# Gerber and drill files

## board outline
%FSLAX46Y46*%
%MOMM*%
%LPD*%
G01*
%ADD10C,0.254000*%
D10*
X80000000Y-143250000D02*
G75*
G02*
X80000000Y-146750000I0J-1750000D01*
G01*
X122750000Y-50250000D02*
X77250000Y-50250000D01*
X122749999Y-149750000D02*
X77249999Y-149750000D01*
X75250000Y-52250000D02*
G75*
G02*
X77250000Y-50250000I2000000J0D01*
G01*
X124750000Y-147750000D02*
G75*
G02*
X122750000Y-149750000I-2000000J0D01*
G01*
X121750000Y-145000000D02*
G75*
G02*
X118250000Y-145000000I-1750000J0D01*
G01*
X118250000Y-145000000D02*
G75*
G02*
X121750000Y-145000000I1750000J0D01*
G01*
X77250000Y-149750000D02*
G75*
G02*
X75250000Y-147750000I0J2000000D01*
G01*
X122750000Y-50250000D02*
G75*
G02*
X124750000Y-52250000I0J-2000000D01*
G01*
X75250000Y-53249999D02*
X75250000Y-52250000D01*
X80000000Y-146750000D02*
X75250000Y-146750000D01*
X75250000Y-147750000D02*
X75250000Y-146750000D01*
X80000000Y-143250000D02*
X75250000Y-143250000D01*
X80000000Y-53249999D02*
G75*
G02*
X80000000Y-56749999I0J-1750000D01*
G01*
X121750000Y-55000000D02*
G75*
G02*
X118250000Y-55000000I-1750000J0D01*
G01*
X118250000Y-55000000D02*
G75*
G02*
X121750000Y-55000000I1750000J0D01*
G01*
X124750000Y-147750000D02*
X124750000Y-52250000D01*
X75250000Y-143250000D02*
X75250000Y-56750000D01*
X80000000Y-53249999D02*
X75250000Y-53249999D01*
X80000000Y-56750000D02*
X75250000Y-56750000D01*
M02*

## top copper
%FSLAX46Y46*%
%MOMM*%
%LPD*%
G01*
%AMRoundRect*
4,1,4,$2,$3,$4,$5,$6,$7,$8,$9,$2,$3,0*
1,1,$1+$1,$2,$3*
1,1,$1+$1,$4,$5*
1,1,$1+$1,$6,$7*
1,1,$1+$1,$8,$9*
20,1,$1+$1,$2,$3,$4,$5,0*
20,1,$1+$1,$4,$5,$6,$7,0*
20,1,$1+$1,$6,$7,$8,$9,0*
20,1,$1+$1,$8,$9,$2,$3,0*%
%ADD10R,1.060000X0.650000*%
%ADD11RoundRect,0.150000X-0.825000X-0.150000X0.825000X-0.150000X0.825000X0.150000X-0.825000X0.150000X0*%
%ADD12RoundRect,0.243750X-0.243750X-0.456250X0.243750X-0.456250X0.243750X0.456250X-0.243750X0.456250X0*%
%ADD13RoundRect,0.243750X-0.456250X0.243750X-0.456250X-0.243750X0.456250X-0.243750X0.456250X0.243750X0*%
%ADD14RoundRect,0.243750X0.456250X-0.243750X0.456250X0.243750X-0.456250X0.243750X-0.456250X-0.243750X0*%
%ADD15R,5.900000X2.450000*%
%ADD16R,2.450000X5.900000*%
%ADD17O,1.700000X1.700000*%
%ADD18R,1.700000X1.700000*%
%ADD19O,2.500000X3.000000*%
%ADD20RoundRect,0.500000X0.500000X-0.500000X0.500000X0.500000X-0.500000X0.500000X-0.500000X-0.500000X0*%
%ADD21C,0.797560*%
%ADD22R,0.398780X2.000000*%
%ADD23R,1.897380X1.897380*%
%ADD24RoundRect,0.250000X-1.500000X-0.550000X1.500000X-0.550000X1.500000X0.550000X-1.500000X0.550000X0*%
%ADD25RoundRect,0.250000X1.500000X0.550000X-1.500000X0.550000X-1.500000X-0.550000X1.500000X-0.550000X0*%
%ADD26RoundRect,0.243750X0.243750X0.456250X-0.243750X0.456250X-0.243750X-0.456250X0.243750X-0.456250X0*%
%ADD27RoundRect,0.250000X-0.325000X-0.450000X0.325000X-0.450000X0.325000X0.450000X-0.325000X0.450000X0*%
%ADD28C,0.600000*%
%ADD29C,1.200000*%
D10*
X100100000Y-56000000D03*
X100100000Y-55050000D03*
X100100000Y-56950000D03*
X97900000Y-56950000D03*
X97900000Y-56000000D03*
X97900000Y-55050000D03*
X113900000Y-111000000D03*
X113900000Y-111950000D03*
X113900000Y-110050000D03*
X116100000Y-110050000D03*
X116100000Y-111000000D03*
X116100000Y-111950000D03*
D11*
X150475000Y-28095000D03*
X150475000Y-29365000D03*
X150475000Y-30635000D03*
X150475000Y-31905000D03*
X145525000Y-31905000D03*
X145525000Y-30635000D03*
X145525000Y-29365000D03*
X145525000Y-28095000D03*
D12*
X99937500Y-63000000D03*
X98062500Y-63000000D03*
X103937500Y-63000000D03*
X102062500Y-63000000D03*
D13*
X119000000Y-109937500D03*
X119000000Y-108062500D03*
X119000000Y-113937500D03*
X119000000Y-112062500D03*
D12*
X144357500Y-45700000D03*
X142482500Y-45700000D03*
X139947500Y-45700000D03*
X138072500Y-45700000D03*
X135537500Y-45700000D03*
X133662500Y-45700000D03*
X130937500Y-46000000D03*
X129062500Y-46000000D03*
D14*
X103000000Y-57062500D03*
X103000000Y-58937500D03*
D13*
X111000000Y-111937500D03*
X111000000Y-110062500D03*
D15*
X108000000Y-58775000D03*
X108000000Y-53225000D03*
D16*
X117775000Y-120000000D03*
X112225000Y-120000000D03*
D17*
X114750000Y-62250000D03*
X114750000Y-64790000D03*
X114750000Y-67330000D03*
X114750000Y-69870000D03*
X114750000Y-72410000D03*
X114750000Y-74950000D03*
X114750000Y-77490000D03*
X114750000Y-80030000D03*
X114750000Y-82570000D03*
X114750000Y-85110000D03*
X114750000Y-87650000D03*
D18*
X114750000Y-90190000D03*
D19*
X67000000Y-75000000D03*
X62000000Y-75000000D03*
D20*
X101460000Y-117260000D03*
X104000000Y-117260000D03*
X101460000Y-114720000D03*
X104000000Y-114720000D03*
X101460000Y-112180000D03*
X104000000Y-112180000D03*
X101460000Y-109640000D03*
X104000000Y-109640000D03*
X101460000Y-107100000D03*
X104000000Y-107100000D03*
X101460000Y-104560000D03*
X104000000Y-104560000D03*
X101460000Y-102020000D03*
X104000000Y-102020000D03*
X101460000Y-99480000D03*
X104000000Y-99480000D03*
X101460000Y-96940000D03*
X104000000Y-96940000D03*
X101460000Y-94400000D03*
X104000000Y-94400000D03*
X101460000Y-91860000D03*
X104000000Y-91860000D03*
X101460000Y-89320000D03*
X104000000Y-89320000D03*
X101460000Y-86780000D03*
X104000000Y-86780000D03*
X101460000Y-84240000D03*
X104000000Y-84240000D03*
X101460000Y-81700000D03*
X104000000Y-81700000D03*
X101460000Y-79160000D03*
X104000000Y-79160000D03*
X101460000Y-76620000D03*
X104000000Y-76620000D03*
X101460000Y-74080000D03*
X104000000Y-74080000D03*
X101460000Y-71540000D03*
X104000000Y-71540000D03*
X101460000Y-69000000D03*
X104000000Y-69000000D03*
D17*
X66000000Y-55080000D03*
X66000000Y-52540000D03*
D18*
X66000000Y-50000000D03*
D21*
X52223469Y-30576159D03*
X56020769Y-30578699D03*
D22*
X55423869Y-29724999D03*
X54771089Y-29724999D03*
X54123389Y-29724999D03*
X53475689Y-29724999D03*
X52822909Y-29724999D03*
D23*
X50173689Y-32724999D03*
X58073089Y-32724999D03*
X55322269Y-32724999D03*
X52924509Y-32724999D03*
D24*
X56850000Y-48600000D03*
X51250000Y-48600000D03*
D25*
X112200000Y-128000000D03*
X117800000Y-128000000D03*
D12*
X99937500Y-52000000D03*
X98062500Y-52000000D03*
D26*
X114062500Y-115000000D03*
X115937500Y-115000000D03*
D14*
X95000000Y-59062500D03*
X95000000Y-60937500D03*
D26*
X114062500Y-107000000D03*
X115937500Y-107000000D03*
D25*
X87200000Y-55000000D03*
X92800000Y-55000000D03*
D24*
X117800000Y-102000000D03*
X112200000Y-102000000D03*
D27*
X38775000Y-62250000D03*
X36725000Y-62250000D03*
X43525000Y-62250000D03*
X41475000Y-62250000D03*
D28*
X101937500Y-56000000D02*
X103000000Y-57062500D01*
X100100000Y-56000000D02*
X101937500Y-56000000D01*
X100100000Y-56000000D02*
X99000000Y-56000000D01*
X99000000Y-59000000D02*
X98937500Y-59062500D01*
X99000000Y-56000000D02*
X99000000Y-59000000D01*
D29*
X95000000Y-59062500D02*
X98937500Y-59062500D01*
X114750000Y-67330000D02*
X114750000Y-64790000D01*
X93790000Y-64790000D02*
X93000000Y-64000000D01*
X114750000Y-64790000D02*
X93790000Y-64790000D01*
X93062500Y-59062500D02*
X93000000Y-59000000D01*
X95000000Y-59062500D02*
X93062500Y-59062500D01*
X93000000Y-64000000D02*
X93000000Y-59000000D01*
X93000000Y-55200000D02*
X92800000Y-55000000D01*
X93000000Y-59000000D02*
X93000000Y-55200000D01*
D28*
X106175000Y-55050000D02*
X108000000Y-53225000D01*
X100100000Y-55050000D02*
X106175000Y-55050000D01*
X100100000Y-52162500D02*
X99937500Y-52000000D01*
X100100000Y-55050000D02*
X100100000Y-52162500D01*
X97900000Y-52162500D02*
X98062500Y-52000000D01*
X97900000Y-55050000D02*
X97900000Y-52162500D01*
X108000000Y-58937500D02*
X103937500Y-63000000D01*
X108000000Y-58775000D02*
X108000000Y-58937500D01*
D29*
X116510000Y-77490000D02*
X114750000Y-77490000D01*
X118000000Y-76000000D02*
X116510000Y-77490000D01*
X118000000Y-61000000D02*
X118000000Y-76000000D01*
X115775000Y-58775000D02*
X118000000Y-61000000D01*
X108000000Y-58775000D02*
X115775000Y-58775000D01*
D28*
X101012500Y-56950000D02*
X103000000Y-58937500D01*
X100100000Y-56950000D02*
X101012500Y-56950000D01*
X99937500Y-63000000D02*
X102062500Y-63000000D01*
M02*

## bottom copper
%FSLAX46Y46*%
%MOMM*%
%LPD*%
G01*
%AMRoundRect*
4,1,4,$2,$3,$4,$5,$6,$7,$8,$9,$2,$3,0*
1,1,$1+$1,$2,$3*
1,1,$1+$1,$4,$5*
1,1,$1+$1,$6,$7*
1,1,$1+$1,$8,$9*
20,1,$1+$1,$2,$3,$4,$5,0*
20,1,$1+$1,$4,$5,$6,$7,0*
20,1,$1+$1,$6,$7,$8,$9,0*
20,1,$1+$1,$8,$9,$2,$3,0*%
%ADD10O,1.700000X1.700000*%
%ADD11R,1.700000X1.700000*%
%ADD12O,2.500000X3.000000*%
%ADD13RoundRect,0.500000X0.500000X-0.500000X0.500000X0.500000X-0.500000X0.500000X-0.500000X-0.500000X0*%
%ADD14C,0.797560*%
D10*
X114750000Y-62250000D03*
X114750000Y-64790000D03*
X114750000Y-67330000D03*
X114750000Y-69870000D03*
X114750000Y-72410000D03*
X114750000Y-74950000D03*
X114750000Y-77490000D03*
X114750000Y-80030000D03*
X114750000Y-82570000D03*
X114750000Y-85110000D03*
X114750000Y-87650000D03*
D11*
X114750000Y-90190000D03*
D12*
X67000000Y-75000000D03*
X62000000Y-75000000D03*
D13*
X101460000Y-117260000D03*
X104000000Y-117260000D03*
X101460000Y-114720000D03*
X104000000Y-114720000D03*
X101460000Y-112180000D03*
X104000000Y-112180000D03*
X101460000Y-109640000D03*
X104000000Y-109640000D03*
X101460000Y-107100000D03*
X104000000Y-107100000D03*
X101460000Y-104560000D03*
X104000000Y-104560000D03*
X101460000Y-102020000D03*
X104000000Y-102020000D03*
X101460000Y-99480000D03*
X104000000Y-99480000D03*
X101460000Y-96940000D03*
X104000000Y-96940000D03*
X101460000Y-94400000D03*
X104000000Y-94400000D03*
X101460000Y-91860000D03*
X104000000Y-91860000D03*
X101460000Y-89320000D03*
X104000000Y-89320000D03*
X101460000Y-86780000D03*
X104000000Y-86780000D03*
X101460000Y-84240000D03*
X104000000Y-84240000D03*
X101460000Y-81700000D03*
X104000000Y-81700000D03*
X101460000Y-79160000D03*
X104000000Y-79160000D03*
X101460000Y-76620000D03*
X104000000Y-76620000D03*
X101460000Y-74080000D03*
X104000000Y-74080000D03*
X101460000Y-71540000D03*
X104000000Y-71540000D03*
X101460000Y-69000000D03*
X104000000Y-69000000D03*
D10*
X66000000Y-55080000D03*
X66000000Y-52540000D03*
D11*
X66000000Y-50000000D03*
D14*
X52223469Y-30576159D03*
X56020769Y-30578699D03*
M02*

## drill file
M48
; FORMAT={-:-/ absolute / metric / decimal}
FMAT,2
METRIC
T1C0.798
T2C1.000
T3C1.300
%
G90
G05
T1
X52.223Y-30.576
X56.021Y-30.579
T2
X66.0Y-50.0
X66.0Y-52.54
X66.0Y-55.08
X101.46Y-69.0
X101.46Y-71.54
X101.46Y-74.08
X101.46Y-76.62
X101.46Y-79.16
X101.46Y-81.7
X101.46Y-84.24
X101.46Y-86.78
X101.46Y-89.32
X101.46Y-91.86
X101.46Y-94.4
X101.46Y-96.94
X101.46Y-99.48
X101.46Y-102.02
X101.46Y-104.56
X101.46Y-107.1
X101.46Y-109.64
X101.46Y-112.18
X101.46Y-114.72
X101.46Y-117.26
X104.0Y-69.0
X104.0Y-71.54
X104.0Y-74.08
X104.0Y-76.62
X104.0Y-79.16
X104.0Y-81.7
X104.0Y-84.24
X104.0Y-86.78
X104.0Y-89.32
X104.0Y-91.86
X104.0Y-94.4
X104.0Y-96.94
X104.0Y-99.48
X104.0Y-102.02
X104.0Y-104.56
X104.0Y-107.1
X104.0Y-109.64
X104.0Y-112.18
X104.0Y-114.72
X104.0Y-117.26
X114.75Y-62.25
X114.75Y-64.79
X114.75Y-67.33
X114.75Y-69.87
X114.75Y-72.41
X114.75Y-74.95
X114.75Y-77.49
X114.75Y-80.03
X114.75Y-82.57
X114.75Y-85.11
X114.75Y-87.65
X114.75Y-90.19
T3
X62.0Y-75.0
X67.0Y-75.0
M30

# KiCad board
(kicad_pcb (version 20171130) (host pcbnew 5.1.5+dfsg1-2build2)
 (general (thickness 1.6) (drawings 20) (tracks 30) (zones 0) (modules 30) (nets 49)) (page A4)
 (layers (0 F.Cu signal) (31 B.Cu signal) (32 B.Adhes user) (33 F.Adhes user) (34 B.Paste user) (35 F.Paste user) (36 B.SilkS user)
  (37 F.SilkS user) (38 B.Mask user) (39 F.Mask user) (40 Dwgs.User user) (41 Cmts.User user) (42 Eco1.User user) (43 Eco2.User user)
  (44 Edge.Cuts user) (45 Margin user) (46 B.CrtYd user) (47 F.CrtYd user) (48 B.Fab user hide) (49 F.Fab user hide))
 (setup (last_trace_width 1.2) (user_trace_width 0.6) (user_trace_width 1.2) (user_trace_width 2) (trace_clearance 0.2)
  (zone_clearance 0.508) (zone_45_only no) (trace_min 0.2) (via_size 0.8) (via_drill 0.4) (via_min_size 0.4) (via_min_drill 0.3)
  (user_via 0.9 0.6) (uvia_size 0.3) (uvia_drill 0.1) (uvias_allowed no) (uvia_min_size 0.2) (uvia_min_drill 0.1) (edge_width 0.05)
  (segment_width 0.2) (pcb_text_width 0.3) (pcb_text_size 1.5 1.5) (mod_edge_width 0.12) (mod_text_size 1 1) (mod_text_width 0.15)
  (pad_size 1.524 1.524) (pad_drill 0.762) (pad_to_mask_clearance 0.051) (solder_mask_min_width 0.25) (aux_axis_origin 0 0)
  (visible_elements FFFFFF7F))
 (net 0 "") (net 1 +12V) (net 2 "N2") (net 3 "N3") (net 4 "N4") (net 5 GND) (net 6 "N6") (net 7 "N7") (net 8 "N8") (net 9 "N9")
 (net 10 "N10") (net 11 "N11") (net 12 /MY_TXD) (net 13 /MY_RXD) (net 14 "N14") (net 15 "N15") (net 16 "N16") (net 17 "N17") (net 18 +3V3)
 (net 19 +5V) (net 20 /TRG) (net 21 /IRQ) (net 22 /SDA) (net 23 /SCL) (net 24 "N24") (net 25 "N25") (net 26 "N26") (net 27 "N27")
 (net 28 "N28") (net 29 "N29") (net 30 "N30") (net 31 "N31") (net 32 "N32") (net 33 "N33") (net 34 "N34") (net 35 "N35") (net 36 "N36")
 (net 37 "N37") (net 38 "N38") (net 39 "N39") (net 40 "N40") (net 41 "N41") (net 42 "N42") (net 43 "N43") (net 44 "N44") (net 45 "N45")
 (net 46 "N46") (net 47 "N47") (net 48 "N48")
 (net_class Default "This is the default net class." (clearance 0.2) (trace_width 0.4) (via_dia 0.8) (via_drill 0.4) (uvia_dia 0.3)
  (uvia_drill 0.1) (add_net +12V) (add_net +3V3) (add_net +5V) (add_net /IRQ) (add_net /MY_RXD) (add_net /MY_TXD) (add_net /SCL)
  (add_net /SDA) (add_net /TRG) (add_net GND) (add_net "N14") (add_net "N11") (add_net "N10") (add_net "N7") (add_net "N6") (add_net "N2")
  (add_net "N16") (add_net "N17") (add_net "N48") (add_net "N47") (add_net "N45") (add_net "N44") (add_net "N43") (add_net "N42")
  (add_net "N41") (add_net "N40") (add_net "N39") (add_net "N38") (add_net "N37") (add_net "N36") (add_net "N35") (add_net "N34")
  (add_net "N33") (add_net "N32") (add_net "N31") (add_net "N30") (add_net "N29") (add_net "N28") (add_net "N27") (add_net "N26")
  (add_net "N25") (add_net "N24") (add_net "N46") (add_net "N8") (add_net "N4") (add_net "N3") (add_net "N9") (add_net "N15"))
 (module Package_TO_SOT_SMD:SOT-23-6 (layer F.Cu) (at 99 56)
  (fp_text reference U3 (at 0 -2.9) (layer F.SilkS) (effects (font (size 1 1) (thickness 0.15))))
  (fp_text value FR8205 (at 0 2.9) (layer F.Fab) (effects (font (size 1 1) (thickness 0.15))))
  (pad 5 smd rect (at 1.1 0) (size 1.06 0.65) (layers F.Cu F.Paste F.Mask) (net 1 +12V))
  (pad 6 smd rect (at 1.1 -0.95) (size 1.06 0.65) (layers F.Cu F.Paste F.Mask) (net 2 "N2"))
  (pad 4 smd rect (at 1.1 0.95) (size 1.06 0.65) (layers F.Cu F.Paste F.Mask) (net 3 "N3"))
  (pad 3 smd rect (at -1.1 0.95) (size 1.06 0.65) (layers F.Cu F.Paste F.Mask) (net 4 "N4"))
  (pad 2 smd rect (at -1.1 0) (size 1.06 0.65) (layers F.Cu F.Paste F.Mask) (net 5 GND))
  (pad 1 smd rect (at -1.1 -0.95) (size 1.06 0.65) (layers F.Cu F.Paste F.Mask) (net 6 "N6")))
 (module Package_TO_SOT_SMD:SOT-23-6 (layer F.Cu) (at 115 111 180)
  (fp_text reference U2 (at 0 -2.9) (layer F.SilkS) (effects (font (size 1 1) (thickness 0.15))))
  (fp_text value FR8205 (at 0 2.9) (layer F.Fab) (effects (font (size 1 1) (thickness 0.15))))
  (pad 5 smd rect (at 1.1 0 180) (size 1.06 0.65) (layers F.Cu F.Paste F.Mask) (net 1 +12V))
  (pad 6 smd rect (at 1.1 -0.95 180) (size 1.06 0.65) (layers F.Cu F.Paste F.Mask) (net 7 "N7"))
  (pad 4 smd rect (at 1.1 0.95 180) (size 1.06 0.65) (layers F.Cu F.Paste F.Mask) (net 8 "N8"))
  (pad 3 smd rect (at -1.1 0.95 180) (size 1.06 0.65) (layers F.Cu F.Paste F.Mask) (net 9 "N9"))
  (pad 2 smd rect (at -1.1 0 180) (size 1.06 0.65) (layers F.Cu F.Paste F.Mask) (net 5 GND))
  (pad 1 smd rect (at -1.1 -0.95 180) (size 1.06 0.65) (layers F.Cu F.Paste F.Mask) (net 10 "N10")))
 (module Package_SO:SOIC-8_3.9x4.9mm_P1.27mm (layer F.Cu) (at 148 30)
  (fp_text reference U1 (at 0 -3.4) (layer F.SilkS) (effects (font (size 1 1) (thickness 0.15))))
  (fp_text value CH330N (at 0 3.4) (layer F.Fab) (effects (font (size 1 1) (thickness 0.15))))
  (pad 8 smd roundrect (at 2.475 -1.905) (size 1.95 0.6) (layers F.Cu F.Paste F.Mask) (roundrect_rratio 0.25) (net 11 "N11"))
  (pad 7 smd roundrect (at 2.475 -0.635) (size 1.95 0.6) (layers F.Cu F.Paste F.Mask) (roundrect_rratio 0.25) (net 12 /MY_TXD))
  (pad 6 smd roundrect (at 2.475 0.635) (size 1.95 0.6) (layers F.Cu F.Paste F.Mask) (roundrect_rratio 0.25) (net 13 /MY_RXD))
  (pad 5 smd roundrect (at 2.475 1.905) (size 1.95 0.6) (layers F.Cu F.Paste F.Mask) (roundrect_rratio 0.25) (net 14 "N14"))
  (pad 4 smd roundrect (at -2.475 1.905) (size 1.95 0.6) (layers F.Cu F.Paste F.Mask) (roundrect_rratio 0.25) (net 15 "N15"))
  (pad 3 smd roundrect (at -2.475 0.635) (size 1.95 0.6) (layers F.Cu F.Paste F.Mask) (roundrect_rratio 0.25) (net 5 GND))
  (pad 2 smd roundrect (at -2.475 -0.635) (size 1.95 0.6) (layers F.Cu F.Paste F.Mask) (roundrect_rratio 0.25) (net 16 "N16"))
  (pad 1 smd roundrect (at -2.475 -1.905) (size 1.95 0.6) (layers F.Cu F.Paste F.Mask) (roundrect_rratio 0.25) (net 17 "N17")))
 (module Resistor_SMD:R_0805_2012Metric (layer F.Cu) (at 99 63)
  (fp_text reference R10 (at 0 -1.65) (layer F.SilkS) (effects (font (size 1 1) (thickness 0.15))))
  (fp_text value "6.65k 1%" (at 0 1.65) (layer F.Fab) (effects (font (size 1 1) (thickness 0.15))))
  (pad 2 smd roundrect (at 0.9375 0) (size 0.975 1.4) (layers F.Cu F.Paste F.Mask) (roundrect_rratio 0.25) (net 4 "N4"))
  (pad 1 smd roundrect (at -0.9375 0) (size 0.975 1.4) (layers F.Cu F.Paste F.Mask) (roundrect_rratio 0.25) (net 5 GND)))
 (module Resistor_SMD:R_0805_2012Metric (layer F.Cu) (at 103 63)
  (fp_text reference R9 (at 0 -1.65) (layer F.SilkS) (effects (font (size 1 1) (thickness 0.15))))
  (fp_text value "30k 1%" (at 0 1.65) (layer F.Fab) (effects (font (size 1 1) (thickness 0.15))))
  (pad 2 smd roundrect (at 0.9375 0) (size 0.975 1.4) (layers F.Cu F.Paste F.Mask) (roundrect_rratio 0.25) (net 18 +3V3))
  (pad 1 smd roundrect (at -0.9375 0) (size 0.975 1.4) (layers F.Cu F.Paste F.Mask) (roundrect_rratio 0.25) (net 4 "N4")))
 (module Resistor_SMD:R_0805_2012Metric (layer F.Cu) (at 119 109 270)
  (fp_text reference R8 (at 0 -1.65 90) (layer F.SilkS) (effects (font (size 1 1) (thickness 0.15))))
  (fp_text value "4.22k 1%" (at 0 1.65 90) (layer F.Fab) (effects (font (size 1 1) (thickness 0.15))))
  (pad 2 smd roundrect (at 0.9375 0 270) (size 0.975 1.4) (layers F.Cu F.Paste F.Mask) (roundrect_rratio 0.25) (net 9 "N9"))
  (pad 1 smd roundrect (at -0.9375 0 270) (size 0.975 1.4) (layers F.Cu F.Paste F.Mask) (roundrect_rratio 0.25) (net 5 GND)))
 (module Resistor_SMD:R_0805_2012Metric (layer F.Cu) (at 119 113 270)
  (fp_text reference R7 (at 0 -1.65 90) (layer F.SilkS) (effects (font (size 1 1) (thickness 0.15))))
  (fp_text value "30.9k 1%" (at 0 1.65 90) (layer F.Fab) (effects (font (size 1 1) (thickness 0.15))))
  (pad 2 smd roundrect (at 0.9375 0 270) (size 0.975 1.4) (layers F.Cu F.Paste F.Mask) (roundrect_rratio 0.25) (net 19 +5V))
  (pad 1 smd roundrect (at -0.9375 0 270) (size 0.975 1.4) (layers F.Cu F.Paste F.Mask) (roundrect_rratio 0.25) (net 9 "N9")))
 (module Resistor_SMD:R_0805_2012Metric (layer F.Cu) (at 143.42 45.7)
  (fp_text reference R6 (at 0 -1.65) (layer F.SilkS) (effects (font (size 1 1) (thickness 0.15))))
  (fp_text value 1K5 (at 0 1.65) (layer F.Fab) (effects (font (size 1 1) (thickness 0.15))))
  (pad 2 smd roundrect (at 0.9375 0) (size 0.975 1.4) (layers F.Cu F.Paste F.Mask) (roundrect_rratio 0.25) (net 18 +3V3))
  (pad 1 smd roundrect (at -0.9375 0) (size 0.975 1.4) (layers F.Cu F.Paste F.Mask) (roundrect_rratio 0.25) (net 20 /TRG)))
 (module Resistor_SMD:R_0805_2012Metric (layer F.Cu) (at 139.01 45.7)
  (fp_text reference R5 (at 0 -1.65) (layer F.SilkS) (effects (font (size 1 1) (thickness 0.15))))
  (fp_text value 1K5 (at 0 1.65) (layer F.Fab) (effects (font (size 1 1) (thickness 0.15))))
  (pad 2 smd roundrect (at 0.9375 0) (size 0.975 1.4) (layers F.Cu F.Paste F.Mask) (roundrect_rratio 0.25) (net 18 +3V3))
  (pad 1 smd roundrect (at -0.9375 0) (size 0.975 1.4) (layers F.Cu F.Paste F.Mask) (roundrect_rratio 0.25) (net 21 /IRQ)))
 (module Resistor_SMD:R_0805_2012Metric (layer F.Cu) (at 134.6 45.7)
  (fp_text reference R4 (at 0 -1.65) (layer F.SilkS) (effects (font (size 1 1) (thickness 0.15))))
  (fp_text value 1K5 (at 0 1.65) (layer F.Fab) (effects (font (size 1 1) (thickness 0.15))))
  (pad 2 smd roundrect (at 0.9375 0) (size 0.975 1.4) (layers F.Cu F.Paste F.Mask) (roundrect_rratio 0.25) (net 18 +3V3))
  (pad 1 smd roundrect (at -0.9375 0) (size 0.975 1.4) (layers F.Cu F.Paste F.Mask) (roundrect_rratio 0.25) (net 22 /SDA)))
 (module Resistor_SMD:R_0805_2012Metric (layer F.Cu) (at 130 46)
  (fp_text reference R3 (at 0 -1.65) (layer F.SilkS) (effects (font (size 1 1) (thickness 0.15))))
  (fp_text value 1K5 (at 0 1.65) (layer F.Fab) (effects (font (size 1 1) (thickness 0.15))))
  (pad 2 smd roundrect (at 0.9375 0) (size 0.975 1.4) (layers F.Cu F.Paste F.Mask) (roundrect_rratio 0.25) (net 18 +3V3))
  (pad 1 smd roundrect (at -0.9375 0) (size 0.975 1.4) (layers F.Cu F.Paste F.Mask) (roundrect_rratio 0.25) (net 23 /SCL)))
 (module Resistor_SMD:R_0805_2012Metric (layer F.Cu) (at 103 58 90)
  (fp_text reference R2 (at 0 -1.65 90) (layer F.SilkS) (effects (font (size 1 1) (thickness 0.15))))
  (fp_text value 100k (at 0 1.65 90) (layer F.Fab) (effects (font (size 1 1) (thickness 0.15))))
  (pad 2 smd roundrect (at 0.9375 0 90) (size 0.975 1.4) (layers F.Cu F.Paste F.Mask) (roundrect_rratio 0.25) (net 1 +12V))
  (pad 1 smd roundrect (at -0.9375 0 90) (size 0.975 1.4) (layers F.Cu F.Paste F.Mask) (roundrect_rratio 0.25) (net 3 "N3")))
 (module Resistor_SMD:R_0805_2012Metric (layer F.Cu) (at 111 111 270)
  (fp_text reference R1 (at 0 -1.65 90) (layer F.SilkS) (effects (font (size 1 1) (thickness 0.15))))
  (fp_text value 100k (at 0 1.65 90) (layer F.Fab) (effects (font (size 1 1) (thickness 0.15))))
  (pad 2 smd roundrect (at 0.9375 0 270) (size 0.975 1.4) (layers F.Cu F.Paste F.Mask) (roundrect_rratio 0.25) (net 1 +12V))
  (pad 1 smd roundrect (at -0.9375 0 270) (size 0.975 1.4) (layers F.Cu F.Paste F.Mask) (roundrect_rratio 0.25) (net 8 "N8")))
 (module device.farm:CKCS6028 (layer F.Cu) (at 108 56 270)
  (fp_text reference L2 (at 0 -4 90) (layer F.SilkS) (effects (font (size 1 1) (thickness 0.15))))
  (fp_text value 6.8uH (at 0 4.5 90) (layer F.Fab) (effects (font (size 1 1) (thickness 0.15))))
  (pad 2 smd rect (at 2.775 0 270) (size 2.45 5.9) (layers F.Cu F.Paste F.Mask) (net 18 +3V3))
  (pad 1 smd rect (at -2.775 0 270) (size 2.45 5.9) (layers F.Cu F.Paste F.Mask) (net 2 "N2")))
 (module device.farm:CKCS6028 (layer F.Cu) (at 115 120)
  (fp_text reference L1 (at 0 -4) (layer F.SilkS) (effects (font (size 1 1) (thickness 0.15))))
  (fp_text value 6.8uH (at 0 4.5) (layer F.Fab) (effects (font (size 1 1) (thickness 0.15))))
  (pad 2 smd rect (at 2.775 0) (size 2.45 5.9) (layers F.Cu F.Paste F.Mask) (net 19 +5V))
  (pad 1 smd rect (at -2.775 0) (size 2.45 5.9) (layers F.Cu F.Paste F.Mask) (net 7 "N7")))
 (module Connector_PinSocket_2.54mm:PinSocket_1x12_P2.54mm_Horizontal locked (layer F.Cu) (at 114.75 90.19 180)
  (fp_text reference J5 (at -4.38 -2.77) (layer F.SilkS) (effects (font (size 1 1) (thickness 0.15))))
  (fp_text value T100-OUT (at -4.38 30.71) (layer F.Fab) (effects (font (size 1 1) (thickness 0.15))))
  (pad 12 thru_hole oval (at 0 27.94 180) (size 1.7 1.7) (drill 1) (layers *.Cu *.Mask) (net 5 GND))
  (pad 11 thru_hole oval (at 0 25.4 180) (size 1.7 1.7) (drill 1) (layers *.Cu *.Mask) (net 1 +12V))
  (pad 10 thru_hole oval (at 0 22.86 180) (size 1.7 1.7) (drill 1) (layers *.Cu *.Mask) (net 1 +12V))
  (pad 9 thru_hole oval (at 0 20.32 180) (size 1.7 1.7) (drill 1) (layers *.Cu *.Mask) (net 5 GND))
  (pad 8 thru_hole oval (at 0 17.78 180) (size 1.7 1.7) (drill 1) (layers *.Cu *.Mask) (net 19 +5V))
  (pad 7 thru_hole oval (at 0 15.24 180) (size 1.7 1.7) (drill 1) (layers *.Cu *.Mask) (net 5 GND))
  (pad 6 thru_hole oval (at 0 12.7 180) (size 1.7 1.7) (drill 1) (layers *.Cu *.Mask) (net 18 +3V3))
  (pad 5 thru_hole oval (at 0 10.16 180) (size 1.7 1.7) (drill 1) (layers *.Cu *.Mask) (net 20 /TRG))
  (pad 4 thru_hole oval (at 0 7.62 180) (size 1.7 1.7) (drill 1) (layers *.Cu *.Mask) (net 21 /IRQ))
  (pad 3 thru_hole oval (at 0 5.08 180) (size 1.7 1.7) (drill 1) (layers *.Cu *.Mask) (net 22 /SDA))
  (pad 2 thru_hole oval (at 0 2.54 180) (size 1.7 1.7) (drill 1) (layers *.Cu *.Mask) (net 23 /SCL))
  (pad 1 thru_hole rect (at 0 0 180) (size 1.7 1.7) (drill 1) (layers *.Cu *.Mask) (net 5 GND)))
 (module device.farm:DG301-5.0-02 (layer F.Cu) (at 62 75)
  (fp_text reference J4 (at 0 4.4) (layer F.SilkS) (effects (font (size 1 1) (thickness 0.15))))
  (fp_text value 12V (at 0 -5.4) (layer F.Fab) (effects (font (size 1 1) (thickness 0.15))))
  (pad 2 thru_hole oval (at 5 0) (size 2.5 3) (drill 1.3) (layers *.Cu *.Mask F.SilkS) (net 1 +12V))
  (pad 1 thru_hole oval (at 0 0) (size 2.5 3) (drill 1.3) (layers *.Cu *.Mask F.SilkS) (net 5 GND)))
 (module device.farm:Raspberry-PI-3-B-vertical (layer F.Cu) (at 104 69 90)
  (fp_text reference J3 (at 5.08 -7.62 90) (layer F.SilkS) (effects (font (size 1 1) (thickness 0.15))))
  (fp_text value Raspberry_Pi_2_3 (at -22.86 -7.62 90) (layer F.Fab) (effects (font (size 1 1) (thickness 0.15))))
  (pad 40 thru_hole roundrect (at -48.26 -2.54 90) (size 2 2) (drill 1) (layers *.Cu *.Mask) (roundrect_rratio 0.25) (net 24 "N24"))
  (pad 39 thru_hole roundrect (at -48.26 0 90) (size 2 2) (drill 1) (layers *.Cu *.Mask) (roundrect_rratio 0.25) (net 5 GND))
  (pad 38 thru_hole roundrect (at -45.72 -2.54 90) (size 2 2) (drill 1) (layers *.Cu *.Mask) (roundrect_rratio 0.25) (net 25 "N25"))
  (pad 37 thru_hole roundrect (at -45.72 0 90) (size 2 2) (drill 1) (layers *.Cu *.Mask) (roundrect_rratio 0.25) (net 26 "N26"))
  (pad 36 thru_hole roundrect (at -43.18 -2.54 90) (size 2 2) (drill 1) (layers *.Cu *.Mask) (roundrect_rratio 0.25) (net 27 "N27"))
  (pad 35 thru_hole roundrect (at -43.18 0 90) (size 2 2) (drill 1) (layers *.Cu *.Mask) (roundrect_rratio 0.25) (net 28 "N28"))
  (pad 34 thru_hole roundrect (at -40.64 -2.54 90) (size 2 2) (drill 1) (layers *.Cu *.Mask) (roundrect_rratio 0.25) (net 5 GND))
  (pad 33 thru_hole roundrect (at -40.64 0 90) (size 2 2) (drill 1) (layers *.Cu *.Mask) (roundrect_rratio 0.25) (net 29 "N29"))
  (pad 32 thru_hole roundrect (at -38.1 -2.54 90) (size 2 2) (drill 1) (layers *.Cu *.Mask) (roundrect_rratio 0.25) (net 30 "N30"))
  (pad 31 thru_hole roundrect (at -38.1 0 90) (size 2 2) (drill 1) (layers *.Cu *.Mask) (roundrect_rratio 0.25) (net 20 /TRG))
  (pad 30 thru_hole roundrect (at -35.56 -2.54 90) (size 2 2) (drill 1) (layers *.Cu *.Mask) (roundrect_rratio 0.25) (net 5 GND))
  (pad 29 thru_hole roundrect (at -35.56 0 90) (size 2 2) (drill 1) (layers *.Cu *.Mask) (roundrect_rratio 0.25) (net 21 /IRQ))
  (pad 28 thru_hole roundrect (at -33.02 -2.54 90) (size 2 2) (drill 1) (layers *.Cu *.Mask) (roundrect_rratio 0.25) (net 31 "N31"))
  (pad 27 thru_hole roundrect (at -33.02 0 90) (size 2 2) (drill 1) (layers *.Cu *.Mask) (roundrect_rratio 0.25) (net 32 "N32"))
  (pad 26 thru_hole roundrect (at -30.48 -2.54 90) (size 2 2) (drill 1) (layers *.Cu *.Mask) (roundrect_rratio 0.25) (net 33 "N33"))
  (pad 25 thru_hole roundrect (at -30.48 0 90) (size 2 2) (drill 1) (layers *.Cu *.Mask) (roundrect_rratio 0.25) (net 5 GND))
  (pad 24 thru_hole roundrect (at -27.94 -2.54 90) (size 2 2) (drill 1) (layers *.Cu *.Mask) (roundrect_rratio 0.25) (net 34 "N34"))
  (pad 23 thru_hole roundrect (at -27.94 0 90) (size 2 2) (drill 1) (layers *.Cu *.Mask) (roundrect_rratio 0.25) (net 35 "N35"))
  (pad 22 thru_hole roundrect (at -25.4 -2.54 90) (size 2 2) (drill 1) (layers *.Cu *.Mask) (roundrect_rratio 0.25) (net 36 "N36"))
  (pad 21 thru_hole roundrect (at -25.4 0 90) (size 2 2) (drill 1) (layers *.Cu *.Mask) (roundrect_rratio 0.25) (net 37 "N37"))
  (pad 20 thru_hole roundrect (at -22.86 -2.54 90) (size 2 2) (drill 1) (layers *.Cu *.Mask) (roundrect_rratio 0.25) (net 5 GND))
  (pad 19 thru_hole roundrect (at -22.86 0 90) (size 2 2) (drill 1) (layers *.Cu *.Mask) (roundrect_rratio 0.25) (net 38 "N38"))
  (pad 18 thru_hole roundrect (at -20.32 -2.54 90) (size 2 2) (drill 1) (layers *.Cu *.Mask) (roundrect_rratio 0.25) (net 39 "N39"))
  (pad 17 thru_hole roundrect (at -20.32 0 90) (size 2 2) (drill 1) (layers *.Cu *.Mask) (roundrect_rratio 0.25) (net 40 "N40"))
  (pad 16 thru_hole roundrect (at -17.78 -2.54 90) (size 2 2) (drill 1) (layers *.Cu *.Mask) (roundrect_rratio 0.25) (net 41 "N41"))
  (pad 15 thru_hole roundrect (at -17.78 0 90) (size 2 2) (drill 1) (layers *.Cu *.Mask) (roundrect_rratio 0.25) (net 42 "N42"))
  (pad 14 thru_hole roundrect (at -15.24 -2.54 90) (size 2 2) (drill 1) (layers *.Cu *.Mask) (roundrect_rratio 0.25) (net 5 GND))
  (pad 13 thru_hole roundrect (at -15.24 0 90) (size 2 2) (drill 1) (layers *.Cu *.Mask) (roundrect_rratio 0.25) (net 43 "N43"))
  (pad 12 thru_hole roundrect (at -12.7 -2.54 90) (size 2 2) (drill 1) (layers *.Cu *.Mask) (roundrect_rratio 0.25) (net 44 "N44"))
  (pad 11 thru_hole roundrect (at -12.7 0 90) (size 2 2) (drill 1) (layers *.Cu *.Mask) (roundrect_rratio 0.25) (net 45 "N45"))
  (pad 10 thru_hole roundrect (at -10.16 -2.54 90) (size 2 2) (drill 1) (layers *.Cu *.Mask) (roundrect_rratio 0.25) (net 13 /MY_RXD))
  (pad 9 thru_hole roundrect (at -10.16 0 90) (size 2 2) (drill 1) (layers *.Cu *.Mask) (roundrect_rratio 0.25) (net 5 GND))
  (pad 8 thru_hole roundrect (at -7.62 -2.54 90) (size 2 2) (drill 1) (layers *.Cu *.Mask) (roundrect_rratio 0.25) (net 12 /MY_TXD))
  (pad 7 thru_hole roundrect (at -7.62 0 90) (size 2 2) (drill 1) (layers *.Cu *.Mask) (roundrect_rratio 0.25) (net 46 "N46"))
  (pad 6 thru_hole roundrect (at -5.08 -2.54 90) (size 2 2) (drill 1) (layers *.Cu *.Mask) (roundrect_rratio 0.25) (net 5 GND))
  (pad 5 thru_hole roundrect (at -5.08 0 90) (size 2 2) (drill 1) (layers *.Cu *.Mask) (roundrect_rratio 0.25) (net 23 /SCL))
  (pad 4 thru_hole roundrect (at -2.54 -2.54 90) (size 2 2) (drill 1) (layers *.Cu *.Mask) (roundrect_rratio 0.25) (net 19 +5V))
  (pad 3 thru_hole roundrect (at -2.54 0 90) (size 2 2) (drill 1) (layers *.Cu *.Mask) (roundrect_rratio 0.25) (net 22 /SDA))
  (pad 2 thru_hole roundrect (at 0 -2.54 90) (size 2 2) (drill 1) (layers *.Cu *.Mask) (roundrect_rratio 0.25) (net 19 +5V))
  (pad 1 thru_hole roundrect (at 0 0 90) (size 2 2) (drill 1) (layers *.Cu *.Mask) (roundrect_rratio 0.25) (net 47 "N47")))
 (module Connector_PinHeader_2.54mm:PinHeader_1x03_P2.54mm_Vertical (layer F.Cu) (at 66 50)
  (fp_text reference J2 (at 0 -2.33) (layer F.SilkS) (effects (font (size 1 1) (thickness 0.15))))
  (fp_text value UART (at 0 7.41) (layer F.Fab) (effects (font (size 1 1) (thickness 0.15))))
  (pad 3 thru_hole oval (at 0 5.08) (size 1.7 1.7) (drill 1) (layers *.Cu *.Mask) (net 13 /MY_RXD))
  (pad 2 thru_hole oval (at 0 2.54) (size 1.7 1.7) (drill 1) (layers *.Cu *.Mask) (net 12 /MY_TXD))
  (pad 1 thru_hole rect (at 0 0) (size 1.7 1.7) (drill 1) (layers *.Cu *.Mask) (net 5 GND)))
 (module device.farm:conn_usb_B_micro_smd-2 (layer F.Cu) (at 54.123389 32.724999)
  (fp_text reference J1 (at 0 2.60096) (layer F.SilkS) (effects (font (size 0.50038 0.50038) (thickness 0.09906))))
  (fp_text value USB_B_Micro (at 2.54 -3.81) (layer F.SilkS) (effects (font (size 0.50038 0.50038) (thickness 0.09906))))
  (pad 1 thru_hole circle (at -1.89992 -2.14884) (size 0.79756 0.79756) (drill 0.79756) (layers *.Cu *.Mask F.SilkS) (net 14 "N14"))
  (pad 5 thru_hole circle (at 1.89738 -2.1463) (size 0.79756 0.79756) (drill 0.79756) (layers *.Cu *.Mask F.SilkS) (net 5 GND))
  (pad 5 smd rect (at 1.30048 -3) (size 0.39878 2) (layers F.Cu F.Paste F.Mask) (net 5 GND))
  (pad 4 smd rect (at 0.6477 -3) (size 0.39878 2) (layers F.Cu F.Paste F.Mask) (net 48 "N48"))
  (pad 3 smd rect (at 0 -3) (size 0.39878 2) (layers F.Cu F.Paste F.Mask) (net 17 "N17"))
  (pad 2 smd rect (at -0.6477 -3) (size 0.39878 2) (layers F.Cu F.Paste F.Mask) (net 16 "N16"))
  (pad 1 smd rect (at -1.30048 -3) (size 0.39878 2) (layers F.Cu F.Paste F.Mask) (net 14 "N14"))
  (pad 6 smd rect (at -3.9497 0) (size 1.89738 1.89738) (layers F.Cu F.Paste F.Mask) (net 5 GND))
  (pad 6 smd rect (at 3.9497 0) (size 1.89738 1.89738) (layers F.Cu F.Paste F.Mask) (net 5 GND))
  (pad 6 smd rect (at 1.19888 0) (size 1.89738 1.89738) (layers F.Cu F.Paste F.Mask) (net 5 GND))
  (pad 6 smd rect (at -1.19888 0) (size 1.89738 1.89738) (layers F.Cu F.Paste F.Mask) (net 5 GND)))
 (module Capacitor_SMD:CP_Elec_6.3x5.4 (layer F.Cu) (at 54.05 48.6)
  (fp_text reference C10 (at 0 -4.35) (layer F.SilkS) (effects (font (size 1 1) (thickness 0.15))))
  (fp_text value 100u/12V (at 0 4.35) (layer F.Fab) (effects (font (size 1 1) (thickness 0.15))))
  (pad 2 smd roundrect (at 2.8 0) (size 3.5 1.6) (layers F.Cu F.Paste F.Mask) (roundrect_rratio 0.15625) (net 5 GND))
  (pad 1 smd roundrect (at -2.8 0) (size 3.5 1.6) (layers F.Cu F.Paste F.Mask) (roundrect_rratio 0.15625) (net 18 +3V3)))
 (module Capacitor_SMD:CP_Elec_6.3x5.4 (layer F.Cu) (at 115 128 180)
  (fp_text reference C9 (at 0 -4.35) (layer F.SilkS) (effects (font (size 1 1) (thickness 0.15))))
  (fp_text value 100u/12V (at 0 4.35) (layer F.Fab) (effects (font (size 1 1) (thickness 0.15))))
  (pad 2 smd roundrect (at 2.8 0 180) (size 3.5 1.6) (layers F.Cu F.Paste F.Mask) (roundrect_rratio 0.15625) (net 5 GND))
  (pad 1 smd roundrect (at -2.8 0 180) (size 3.5 1.6) (layers F.Cu F.Paste F.Mask) (roundrect_rratio 0.15625) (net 19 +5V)))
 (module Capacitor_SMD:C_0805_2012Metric (layer F.Cu) (at 99 52)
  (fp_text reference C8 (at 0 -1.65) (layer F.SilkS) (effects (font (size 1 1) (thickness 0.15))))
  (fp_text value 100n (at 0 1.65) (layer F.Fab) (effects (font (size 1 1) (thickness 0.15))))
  (pad 2 smd roundrect (at 0.9375 0) (size 0.975 1.4) (layers F.Cu F.Paste F.Mask) (roundrect_rratio 0.25) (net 2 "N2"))
  (pad 1 smd roundrect (at -0.9375 0) (size 0.975 1.4) (layers F.Cu F.Paste F.Mask) (roundrect_rratio 0.25) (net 6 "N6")))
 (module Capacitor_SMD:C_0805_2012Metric (layer F.Cu) (at 115 115 180)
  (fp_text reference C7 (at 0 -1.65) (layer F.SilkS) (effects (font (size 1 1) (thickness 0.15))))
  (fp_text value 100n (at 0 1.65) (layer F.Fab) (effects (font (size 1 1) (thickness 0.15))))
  (pad 2 smd roundrect (at 0.9375 0 180) (size 0.975 1.4) (layers F.Cu F.Paste F.Mask) (roundrect_rratio 0.25) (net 7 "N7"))
  (pad 1 smd roundrect (at -0.9375 0 180) (size 0.975 1.4) (layers F.Cu F.Paste F.Mask) (roundrect_rratio 0.25) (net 10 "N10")))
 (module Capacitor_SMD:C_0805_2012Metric (layer F.Cu) (at 95 60 90)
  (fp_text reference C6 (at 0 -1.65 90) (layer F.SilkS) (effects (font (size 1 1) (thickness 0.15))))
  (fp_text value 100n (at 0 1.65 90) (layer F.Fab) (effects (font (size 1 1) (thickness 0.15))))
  (pad 2 smd roundrect (at 0.9375 0 90) (size 0.975 1.4) (layers F.Cu F.Paste F.Mask) (roundrect_rratio 0.25) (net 1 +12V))
  (pad 1 smd roundrect (at -0.9375 0 90) (size 0.975 1.4) (layers F.Cu F.Paste F.Mask) (roundrect_rratio 0.25) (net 5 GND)))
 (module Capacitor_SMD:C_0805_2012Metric (layer F.Cu) (at 115 107 180)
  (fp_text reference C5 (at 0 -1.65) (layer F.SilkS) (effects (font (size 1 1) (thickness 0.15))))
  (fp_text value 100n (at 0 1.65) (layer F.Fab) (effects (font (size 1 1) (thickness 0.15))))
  (pad 2 smd roundrect (at 0.9375 0 180) (size 0.975 1.4) (layers F.Cu F.Paste F.Mask) (roundrect_rratio 0.25) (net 1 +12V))
  (pad 1 smd roundrect (at -0.9375 0 180) (size 0.975 1.4) (layers F.Cu F.Paste F.Mask) (roundrect_rratio 0.25) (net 5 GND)))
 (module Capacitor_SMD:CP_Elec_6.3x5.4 (layer F.Cu) (at 90 55 180)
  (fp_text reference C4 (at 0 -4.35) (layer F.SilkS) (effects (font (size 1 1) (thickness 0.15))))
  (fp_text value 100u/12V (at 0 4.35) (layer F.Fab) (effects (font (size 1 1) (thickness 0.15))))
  (pad 2 smd roundrect (at 2.8 0 180) (size 3.5 1.6) (layers F.Cu F.Paste F.Mask) (roundrect_rratio 0.15625) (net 5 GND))
  (pad 1 smd roundrect (at -2.8 0 180) (size 3.5 1.6) (layers F.Cu F.Paste F.Mask) (roundrect_rratio 0.15625) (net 1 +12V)))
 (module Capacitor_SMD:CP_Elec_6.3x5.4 (layer F.Cu) (at 115 102)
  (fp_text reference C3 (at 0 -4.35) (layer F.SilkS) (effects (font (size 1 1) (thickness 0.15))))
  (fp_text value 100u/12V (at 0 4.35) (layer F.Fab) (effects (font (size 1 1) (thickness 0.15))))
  (pad 2 smd roundrect (at 2.8 0) (size 3.5 1.6) (layers F.Cu F.Paste F.Mask) (roundrect_rratio 0.15625) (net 5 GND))
  (pad 1 smd roundrect (at -2.8 0) (size 3.5 1.6) (layers F.Cu F.Paste F.Mask) (roundrect_rratio 0.15625) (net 1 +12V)))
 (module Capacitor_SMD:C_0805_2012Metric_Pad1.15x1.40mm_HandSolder (layer F.Cu) (at 37.75 62.25)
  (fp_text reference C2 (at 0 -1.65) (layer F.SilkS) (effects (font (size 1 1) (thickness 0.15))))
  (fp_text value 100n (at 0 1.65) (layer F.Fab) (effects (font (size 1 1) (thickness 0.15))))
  (pad 2 smd roundrect (at 1.025 0) (size 1.15 1.4) (layers F.Cu F.Paste F.Mask) (roundrect_rratio 0.217391) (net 5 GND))
  (pad 1 smd roundrect (at -1.025 0) (size 1.15 1.4) (layers F.Cu F.Paste F.Mask) (roundrect_rratio 0.217391) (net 11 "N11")))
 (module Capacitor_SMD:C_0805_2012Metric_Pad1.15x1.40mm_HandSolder (layer F.Cu) (at 42.5 62.25)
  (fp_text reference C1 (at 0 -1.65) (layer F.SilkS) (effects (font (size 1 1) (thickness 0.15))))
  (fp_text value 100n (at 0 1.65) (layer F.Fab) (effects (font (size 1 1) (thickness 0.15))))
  (pad 2 smd roundrect (at 1.025 0) (size 1.15 1.4) (layers F.Cu F.Paste F.Mask) (roundrect_rratio 0.217391) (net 5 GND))
  (pad 1 smd roundrect (at -1.025 0) (size 1.15 1.4) (layers F.Cu F.Paste F.Mask) (roundrect_rratio 0.217391) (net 14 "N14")))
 (gr_arc (start 80 145) (end 80 146.75) (angle -180) (layer Edge.Cuts) (width 0.254))
 (gr_line (start 122.75 50.25) (end 77.25 50.25) (layer Edge.Cuts) (width 0.254))
 (gr_line (start 122.749999 149.75) (end 77.249999 149.75) (layer Edge.Cuts) (width 0.254))
 (gr_arc (start 77.25 52.25) (end 77.25 50.25) (angle -90) (layer Edge.Cuts) (width 0.254))
 (gr_arc (start 122.75 147.75) (end 122.75 149.75) (angle -90) (layer Edge.Cuts) (width 0.254))
 (gr_circle (center 120 145) (end 121.75 145) (layer Edge.Cuts) (width 0.254))
 (gr_arc (start 77.25 147.75) (end 75.25 147.75) (angle -90) (layer Edge.Cuts) (width 0.254))
 (gr_arc (start 122.75 52.25) (end 124.75 52.25) (angle -90) (layer Edge.Cuts) (width 0.254))
 (gr_line (start 75.25 53.249999) (end 75.25 52.25) (layer Edge.Cuts) (width 0.254))
 (gr_line (start 80 146.75) (end 75.25 146.75) (layer Edge.Cuts) (width 0.254))
 (gr_line (start 75.25 147.75) (end 75.25 146.75) (layer Edge.Cuts) (width 0.254))
 (gr_line (start 80 143.25) (end 75.25 143.25) (layer Edge.Cuts) (width 0.254))
 (gr_arc (start 80 54.999999) (end 80 56.749999) (angle -180) (layer Edge.Cuts) (width 0.254))
 (gr_circle (center 120 55) (end 121.75 55) (layer Edge.Cuts) (width 0.254))
 (gr_line (start 124.75 147.75) (end 124.75 52.25) (layer Edge.Cuts) (width 0.254))
 (gr_line (start 75.25 143.25) (end 75.25 56.75) (layer Edge.Cuts) (width 0.254))
 (gr_line (start 80 53.249999) (end 75.25 53.249999) (layer Edge.Cuts) (width 0.254))
 (gr_line (start 80 56.75) (end 75.25 56.75) (layer Edge.Cuts) (width 0.254))
 (segment (start 101.9375 56) (end 103 57.0625) (width 0.6) (layer F.Cu) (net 1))
 (segment (start 100.1 56) (end 101.9375 56) (width 0.6) (layer F.Cu) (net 1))
 (segment (start 100.1 56) (end 99 56) (width 0.6) (layer F.Cu) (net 1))
 (segment (start 99 59) (end 98.9375 59.0625) (width 0.6) (layer F.Cu) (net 1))
 (segment (start 99 56) (end 99 59) (width 0.6) (layer F.Cu) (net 1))
 (segment (start 95 59.0625) (end 98.9375 59.0625) (width 1.2) (layer F.Cu) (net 1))
 (segment (start 114.75 67.33) (end 114.75 64.79) (width 1.2) (layer F.Cu) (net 1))
 (segment (start 93.79 64.79) (end 93 64) (width 1.2) (layer F.Cu) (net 1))
 (segment (start 114.75 64.79) (end 93.79 64.79) (width 1.2) (layer F.Cu) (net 1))
 (segment (start 93.0625 59.0625) (end 93 59) (width 1.2) (layer F.Cu) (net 1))
 (segment (start 95 59.0625) (end 93.0625 59.0625) (width 1.2) (layer F.Cu) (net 1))
 (segment (start 93 64) (end 93 59) (width 1.2) (layer F.Cu) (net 1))
 (segment (start 93 55.2) (end 92.8 55) (width 1.2) (layer F.Cu) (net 1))
 (segment (start 93 59) (end 93 55.2) (width 1.2) (layer F.Cu) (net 1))
 (segment (start 106.175 55.05) (end 108 53.225) (width 0.6) (layer F.Cu) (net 2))
 (segment (start 100.1 55.05) (end 106.175 55.05) (width 0.6) (layer F.Cu) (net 2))
 (segment (start 100.1 52.1625) (end 99.9375 52) (width 0.6) (layer F.Cu) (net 2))
 (segment (start 100.1 55.05) (end 100.1 52.1625) (width 0.6) (layer F.Cu) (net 2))
 (segment (start 97.9 52.1625) (end 98.0625 52) (width 0.6) (layer F.Cu) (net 6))
 (segment (start 97.9 55.05) (end 97.9 52.1625) (width 0.6) (layer F.Cu) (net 6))
 (segment (start 108 58.9375) (end 103.9375 63) (width 0.6) (layer F.Cu) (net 18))
 (segment (start 108 58.775) (end 108 58.9375) (width 0.6) (layer F.Cu) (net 18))
 (segment (start 116.51 77.49) (end 114.75 77.49) (width 1.2) (layer F.Cu) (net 18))
 (segment (start 118 76) (end 116.51 77.49) (width 1.2) (layer F.Cu) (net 18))
 (segment (start 118 61) (end 118 76) (width 1.2) (layer F.Cu) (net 18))
 (segment (start 115.775 58.775) (end 118 61) (width 1.2) (layer F.Cu) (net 18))
 (segment (start 108 58.775) (end 115.775 58.775) (width 1.2) (layer F.Cu) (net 18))
 (segment (start 101.0125 56.95) (end 103 58.9375) (width 0.6) (layer F.Cu) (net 3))
 (segment (start 100.1 56.95) (end 101.0125 56.95) (width 0.6) (layer F.Cu) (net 3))
 (segment (start 99.9375 63) (end 102.0625 63) (width 0.6) (layer F.Cu) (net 4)))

